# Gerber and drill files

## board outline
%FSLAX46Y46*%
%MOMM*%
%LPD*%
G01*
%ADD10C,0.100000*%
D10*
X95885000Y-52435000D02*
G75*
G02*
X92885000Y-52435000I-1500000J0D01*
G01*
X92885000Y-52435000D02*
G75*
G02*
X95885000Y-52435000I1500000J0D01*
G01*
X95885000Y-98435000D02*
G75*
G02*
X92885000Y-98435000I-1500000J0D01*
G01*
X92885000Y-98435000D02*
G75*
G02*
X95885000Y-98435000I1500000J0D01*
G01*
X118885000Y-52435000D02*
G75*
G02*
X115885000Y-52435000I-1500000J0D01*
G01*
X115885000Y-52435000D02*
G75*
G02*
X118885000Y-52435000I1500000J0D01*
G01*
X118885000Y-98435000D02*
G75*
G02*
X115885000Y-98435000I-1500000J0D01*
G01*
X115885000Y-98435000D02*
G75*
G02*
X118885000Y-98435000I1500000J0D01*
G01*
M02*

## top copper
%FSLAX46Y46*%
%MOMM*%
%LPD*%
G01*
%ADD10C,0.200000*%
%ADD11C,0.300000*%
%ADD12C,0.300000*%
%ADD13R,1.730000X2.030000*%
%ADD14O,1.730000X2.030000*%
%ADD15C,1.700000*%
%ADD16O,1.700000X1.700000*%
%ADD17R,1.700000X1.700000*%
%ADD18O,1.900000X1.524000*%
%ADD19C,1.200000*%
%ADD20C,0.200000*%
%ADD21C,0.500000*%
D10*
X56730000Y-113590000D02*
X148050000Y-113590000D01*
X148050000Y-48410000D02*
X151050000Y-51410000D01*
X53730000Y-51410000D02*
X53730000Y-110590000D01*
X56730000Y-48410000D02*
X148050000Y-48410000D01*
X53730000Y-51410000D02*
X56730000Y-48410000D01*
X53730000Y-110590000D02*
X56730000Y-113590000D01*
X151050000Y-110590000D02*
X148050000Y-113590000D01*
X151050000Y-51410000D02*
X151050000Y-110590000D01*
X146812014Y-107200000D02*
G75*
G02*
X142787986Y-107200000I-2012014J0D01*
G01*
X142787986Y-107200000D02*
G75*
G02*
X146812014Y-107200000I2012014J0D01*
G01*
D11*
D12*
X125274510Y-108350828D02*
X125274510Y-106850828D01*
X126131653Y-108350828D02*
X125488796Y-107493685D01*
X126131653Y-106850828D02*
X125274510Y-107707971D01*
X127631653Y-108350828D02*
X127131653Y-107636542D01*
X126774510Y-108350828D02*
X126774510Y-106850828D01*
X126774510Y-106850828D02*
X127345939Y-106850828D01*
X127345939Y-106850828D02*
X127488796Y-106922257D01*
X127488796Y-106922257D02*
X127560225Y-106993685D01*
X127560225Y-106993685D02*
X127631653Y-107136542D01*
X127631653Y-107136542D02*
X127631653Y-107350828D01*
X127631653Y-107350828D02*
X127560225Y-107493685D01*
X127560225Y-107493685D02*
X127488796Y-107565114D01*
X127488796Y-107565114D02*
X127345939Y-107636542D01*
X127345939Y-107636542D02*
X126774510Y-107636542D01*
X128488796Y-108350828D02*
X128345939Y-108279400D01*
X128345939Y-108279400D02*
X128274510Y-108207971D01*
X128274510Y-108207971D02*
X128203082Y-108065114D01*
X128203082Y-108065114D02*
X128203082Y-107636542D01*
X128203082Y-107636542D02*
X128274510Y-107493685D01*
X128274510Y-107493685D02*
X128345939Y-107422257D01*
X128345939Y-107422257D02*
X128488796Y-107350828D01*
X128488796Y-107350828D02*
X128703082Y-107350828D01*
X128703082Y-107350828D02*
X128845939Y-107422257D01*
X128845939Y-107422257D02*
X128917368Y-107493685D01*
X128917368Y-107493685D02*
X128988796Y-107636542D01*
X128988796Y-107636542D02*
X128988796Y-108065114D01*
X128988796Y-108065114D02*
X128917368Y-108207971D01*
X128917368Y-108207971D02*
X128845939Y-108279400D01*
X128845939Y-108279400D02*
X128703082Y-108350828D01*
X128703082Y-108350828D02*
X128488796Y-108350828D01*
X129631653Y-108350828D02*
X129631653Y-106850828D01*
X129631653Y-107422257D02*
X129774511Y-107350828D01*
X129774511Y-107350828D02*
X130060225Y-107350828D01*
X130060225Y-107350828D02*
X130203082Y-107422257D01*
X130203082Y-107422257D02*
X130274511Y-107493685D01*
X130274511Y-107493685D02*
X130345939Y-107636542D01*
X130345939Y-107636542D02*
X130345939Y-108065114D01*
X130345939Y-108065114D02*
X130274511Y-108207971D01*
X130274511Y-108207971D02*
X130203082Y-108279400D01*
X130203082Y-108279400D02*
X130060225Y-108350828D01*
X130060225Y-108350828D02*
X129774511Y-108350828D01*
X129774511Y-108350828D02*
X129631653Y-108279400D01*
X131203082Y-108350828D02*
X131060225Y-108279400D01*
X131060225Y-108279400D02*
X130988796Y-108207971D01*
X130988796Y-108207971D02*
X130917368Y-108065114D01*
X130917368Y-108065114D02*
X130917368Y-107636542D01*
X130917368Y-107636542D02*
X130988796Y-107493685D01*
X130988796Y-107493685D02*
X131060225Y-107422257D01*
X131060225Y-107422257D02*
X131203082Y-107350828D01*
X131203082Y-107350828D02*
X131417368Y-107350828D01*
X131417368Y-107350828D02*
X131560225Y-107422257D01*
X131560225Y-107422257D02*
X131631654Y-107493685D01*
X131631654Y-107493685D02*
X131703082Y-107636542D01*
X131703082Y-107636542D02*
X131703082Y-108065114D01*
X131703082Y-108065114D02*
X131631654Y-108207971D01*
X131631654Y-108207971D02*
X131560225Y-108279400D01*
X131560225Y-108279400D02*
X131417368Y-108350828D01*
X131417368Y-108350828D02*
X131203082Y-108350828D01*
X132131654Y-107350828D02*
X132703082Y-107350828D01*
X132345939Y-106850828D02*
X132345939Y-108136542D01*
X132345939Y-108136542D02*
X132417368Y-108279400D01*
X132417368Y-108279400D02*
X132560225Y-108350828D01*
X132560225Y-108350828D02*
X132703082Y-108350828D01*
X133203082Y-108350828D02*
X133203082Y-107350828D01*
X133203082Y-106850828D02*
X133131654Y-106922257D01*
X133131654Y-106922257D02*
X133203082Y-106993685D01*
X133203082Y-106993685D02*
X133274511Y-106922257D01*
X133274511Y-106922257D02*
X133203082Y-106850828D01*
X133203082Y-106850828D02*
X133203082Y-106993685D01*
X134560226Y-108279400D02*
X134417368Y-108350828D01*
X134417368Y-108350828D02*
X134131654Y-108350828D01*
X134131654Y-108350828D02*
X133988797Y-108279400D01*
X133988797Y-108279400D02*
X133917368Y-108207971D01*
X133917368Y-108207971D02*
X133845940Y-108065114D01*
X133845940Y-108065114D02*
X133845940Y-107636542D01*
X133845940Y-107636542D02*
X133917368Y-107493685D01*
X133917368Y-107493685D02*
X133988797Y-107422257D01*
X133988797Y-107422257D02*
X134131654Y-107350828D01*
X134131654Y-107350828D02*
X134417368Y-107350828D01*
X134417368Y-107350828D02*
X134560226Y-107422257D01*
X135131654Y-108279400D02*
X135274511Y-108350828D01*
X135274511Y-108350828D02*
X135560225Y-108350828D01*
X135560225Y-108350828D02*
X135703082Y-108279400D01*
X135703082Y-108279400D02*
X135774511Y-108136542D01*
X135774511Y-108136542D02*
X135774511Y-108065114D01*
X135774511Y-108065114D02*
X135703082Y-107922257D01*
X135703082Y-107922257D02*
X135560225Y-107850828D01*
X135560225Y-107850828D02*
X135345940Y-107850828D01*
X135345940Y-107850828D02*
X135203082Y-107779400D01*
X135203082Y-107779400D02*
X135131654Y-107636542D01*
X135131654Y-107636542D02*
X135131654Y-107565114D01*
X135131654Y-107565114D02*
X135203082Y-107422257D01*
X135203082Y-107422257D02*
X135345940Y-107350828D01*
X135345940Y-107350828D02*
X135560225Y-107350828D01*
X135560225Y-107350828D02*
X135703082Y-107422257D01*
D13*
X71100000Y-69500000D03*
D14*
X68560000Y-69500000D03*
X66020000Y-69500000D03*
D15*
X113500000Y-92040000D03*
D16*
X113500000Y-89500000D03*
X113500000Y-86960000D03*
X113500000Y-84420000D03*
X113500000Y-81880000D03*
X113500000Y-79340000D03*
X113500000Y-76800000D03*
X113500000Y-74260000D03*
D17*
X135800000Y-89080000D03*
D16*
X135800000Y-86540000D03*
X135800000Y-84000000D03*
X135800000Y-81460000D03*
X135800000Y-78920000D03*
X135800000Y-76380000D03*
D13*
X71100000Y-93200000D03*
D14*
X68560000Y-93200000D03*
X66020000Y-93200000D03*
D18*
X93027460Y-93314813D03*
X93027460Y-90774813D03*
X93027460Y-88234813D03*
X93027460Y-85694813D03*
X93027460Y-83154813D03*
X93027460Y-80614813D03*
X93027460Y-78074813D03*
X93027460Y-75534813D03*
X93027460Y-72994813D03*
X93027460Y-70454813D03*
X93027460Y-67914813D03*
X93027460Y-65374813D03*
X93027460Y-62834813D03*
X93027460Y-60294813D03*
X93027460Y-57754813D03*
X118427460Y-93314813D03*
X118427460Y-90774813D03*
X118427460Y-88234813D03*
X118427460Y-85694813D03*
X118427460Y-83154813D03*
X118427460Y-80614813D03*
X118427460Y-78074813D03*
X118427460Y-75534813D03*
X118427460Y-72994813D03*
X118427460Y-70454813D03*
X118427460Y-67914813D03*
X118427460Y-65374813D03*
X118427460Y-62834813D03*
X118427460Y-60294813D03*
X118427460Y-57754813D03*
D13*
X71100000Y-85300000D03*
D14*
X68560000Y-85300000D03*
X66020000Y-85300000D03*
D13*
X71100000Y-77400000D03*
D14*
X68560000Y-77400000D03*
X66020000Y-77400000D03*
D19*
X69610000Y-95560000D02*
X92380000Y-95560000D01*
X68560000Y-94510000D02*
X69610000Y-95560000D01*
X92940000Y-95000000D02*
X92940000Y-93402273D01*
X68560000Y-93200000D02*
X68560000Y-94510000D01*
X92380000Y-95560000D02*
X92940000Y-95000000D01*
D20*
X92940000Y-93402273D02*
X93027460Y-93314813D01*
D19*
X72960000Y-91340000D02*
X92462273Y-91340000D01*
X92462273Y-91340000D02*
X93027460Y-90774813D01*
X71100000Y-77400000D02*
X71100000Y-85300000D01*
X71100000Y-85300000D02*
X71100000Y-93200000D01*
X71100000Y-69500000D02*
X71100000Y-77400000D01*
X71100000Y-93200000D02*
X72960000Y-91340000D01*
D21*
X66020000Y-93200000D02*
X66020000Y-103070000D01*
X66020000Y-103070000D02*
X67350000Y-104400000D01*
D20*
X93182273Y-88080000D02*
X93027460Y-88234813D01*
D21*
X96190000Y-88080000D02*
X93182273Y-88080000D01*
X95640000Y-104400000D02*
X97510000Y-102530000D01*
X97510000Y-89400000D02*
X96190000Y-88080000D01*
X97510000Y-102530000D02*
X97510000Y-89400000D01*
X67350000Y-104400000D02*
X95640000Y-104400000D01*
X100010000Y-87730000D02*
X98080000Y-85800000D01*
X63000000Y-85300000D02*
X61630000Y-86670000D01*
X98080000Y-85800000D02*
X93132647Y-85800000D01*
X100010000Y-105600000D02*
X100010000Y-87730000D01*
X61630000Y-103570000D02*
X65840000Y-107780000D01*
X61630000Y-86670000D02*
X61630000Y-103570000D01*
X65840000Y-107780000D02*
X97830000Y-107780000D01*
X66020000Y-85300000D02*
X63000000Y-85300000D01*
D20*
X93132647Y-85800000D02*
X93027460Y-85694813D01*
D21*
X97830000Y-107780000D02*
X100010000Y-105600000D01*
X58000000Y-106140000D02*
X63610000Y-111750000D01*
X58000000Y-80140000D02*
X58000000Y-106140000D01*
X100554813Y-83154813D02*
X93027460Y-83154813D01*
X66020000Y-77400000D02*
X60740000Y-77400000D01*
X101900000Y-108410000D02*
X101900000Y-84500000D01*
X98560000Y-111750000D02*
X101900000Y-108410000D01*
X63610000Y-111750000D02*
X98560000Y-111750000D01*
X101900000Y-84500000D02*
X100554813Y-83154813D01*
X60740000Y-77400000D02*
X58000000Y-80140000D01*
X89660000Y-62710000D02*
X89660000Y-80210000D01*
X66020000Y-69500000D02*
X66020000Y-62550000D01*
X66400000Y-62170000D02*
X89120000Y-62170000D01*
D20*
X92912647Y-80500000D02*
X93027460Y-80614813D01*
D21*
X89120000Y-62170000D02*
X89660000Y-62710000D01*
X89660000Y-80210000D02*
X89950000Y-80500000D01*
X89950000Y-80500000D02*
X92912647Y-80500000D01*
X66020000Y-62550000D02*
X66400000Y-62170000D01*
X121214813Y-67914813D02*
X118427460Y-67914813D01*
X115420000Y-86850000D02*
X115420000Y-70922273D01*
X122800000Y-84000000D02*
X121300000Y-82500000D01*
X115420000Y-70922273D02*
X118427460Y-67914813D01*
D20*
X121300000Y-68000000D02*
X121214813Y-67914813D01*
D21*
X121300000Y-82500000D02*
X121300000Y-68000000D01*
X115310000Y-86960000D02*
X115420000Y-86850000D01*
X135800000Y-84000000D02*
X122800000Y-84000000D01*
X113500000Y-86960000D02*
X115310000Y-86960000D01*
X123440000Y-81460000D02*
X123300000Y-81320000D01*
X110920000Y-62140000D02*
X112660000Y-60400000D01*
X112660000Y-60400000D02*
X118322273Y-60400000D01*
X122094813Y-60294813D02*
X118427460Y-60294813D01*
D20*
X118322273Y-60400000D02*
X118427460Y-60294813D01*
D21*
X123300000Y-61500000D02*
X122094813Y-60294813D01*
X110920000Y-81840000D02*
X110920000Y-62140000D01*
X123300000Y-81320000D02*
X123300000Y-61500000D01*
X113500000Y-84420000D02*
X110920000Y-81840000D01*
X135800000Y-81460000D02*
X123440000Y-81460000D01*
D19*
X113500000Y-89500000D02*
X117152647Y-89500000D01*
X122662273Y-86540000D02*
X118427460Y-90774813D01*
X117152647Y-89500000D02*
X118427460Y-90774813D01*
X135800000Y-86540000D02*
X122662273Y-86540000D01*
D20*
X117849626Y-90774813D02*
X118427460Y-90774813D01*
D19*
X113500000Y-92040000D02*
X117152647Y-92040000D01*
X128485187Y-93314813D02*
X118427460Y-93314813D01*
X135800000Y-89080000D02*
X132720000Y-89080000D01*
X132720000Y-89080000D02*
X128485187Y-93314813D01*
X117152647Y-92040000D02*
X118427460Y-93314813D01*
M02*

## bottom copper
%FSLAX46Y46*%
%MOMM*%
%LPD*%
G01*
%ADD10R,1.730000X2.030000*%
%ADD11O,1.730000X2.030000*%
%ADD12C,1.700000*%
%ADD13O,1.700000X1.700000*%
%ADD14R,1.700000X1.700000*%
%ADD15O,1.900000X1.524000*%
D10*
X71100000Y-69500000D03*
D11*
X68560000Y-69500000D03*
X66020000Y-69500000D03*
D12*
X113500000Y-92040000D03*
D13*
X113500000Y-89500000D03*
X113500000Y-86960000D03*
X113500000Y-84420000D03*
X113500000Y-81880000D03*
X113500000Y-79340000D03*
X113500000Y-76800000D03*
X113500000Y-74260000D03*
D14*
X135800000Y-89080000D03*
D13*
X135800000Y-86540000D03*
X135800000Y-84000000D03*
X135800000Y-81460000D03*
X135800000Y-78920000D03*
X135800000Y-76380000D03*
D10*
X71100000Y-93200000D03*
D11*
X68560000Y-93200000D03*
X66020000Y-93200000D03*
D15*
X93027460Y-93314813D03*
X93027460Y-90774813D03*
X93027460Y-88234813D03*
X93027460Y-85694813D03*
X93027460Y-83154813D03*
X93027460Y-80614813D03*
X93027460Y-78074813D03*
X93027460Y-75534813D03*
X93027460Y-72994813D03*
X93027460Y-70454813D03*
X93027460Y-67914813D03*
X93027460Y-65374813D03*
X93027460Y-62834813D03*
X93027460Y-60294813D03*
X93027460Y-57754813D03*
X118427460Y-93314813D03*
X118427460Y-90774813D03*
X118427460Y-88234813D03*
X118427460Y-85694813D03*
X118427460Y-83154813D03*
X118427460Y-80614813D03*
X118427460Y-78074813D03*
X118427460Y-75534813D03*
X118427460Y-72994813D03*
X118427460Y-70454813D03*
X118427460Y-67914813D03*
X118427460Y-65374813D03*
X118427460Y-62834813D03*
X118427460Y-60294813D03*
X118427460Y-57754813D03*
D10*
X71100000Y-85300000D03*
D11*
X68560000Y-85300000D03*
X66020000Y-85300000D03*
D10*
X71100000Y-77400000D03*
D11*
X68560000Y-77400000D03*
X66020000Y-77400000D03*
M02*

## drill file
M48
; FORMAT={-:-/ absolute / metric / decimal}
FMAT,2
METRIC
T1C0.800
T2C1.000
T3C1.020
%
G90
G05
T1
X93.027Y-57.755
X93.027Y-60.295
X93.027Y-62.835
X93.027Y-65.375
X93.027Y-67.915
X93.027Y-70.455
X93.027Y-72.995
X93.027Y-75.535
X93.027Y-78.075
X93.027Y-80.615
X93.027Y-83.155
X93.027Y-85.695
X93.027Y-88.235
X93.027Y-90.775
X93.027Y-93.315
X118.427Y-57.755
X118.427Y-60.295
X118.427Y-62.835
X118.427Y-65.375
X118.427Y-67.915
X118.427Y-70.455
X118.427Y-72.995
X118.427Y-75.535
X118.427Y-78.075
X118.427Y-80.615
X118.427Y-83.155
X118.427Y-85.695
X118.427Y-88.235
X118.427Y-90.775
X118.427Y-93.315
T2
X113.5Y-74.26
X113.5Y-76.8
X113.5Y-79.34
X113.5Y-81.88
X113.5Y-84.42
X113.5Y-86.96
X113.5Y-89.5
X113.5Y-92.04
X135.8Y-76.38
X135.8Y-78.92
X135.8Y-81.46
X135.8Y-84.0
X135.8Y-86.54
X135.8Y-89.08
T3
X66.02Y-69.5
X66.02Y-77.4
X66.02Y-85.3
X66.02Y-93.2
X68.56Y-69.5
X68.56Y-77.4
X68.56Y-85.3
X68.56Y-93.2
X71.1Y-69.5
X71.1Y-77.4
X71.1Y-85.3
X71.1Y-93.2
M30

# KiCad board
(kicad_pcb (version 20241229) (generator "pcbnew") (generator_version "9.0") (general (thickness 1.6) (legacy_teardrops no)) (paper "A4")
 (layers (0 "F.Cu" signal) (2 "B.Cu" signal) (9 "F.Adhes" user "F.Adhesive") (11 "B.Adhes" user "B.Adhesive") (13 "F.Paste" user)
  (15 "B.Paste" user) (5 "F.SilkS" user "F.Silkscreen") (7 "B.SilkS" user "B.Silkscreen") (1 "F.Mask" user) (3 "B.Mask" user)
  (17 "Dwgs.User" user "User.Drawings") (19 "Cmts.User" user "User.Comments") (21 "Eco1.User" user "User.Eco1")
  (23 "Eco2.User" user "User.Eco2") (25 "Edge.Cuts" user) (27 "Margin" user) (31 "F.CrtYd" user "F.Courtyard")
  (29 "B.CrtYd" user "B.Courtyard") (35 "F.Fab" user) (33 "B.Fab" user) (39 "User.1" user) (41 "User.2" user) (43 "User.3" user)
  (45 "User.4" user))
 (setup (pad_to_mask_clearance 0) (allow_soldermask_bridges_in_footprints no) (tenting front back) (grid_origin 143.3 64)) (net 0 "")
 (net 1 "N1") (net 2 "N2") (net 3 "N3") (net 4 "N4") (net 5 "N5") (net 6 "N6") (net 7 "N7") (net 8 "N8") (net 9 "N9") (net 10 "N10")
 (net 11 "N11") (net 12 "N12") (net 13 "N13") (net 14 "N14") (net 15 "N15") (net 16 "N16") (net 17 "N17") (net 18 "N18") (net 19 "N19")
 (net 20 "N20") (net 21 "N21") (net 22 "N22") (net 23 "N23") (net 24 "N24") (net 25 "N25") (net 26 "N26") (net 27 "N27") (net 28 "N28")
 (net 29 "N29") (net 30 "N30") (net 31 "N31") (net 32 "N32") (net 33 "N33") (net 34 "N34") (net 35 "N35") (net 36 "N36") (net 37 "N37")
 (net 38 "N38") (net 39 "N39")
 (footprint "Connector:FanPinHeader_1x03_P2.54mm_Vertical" (layer "F.Cu") (at 71.1 69.5 180)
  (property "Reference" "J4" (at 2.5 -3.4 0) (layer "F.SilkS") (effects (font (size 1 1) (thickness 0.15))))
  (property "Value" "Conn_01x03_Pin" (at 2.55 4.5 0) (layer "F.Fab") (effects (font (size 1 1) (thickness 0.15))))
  (pad "1" thru_hole rect (at 0 0 270) (size 2.03 1.73) (drill 1.02) (layers "*.Cu" "*.Mask") (remove_unused_layers no) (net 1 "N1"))
  (pad "2" thru_hole oval (at 2.54 0 270) (size 2.03 1.73) (drill 1.02) (layers "*.Cu" "*.Mask") (remove_unused_layers no) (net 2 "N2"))
  (pad "3" thru_hole oval (at 5.08 0 270) (size 2.03 1.73) (drill 1.02) (layers "*.Cu" "*.Mask") (remove_unused_layers no) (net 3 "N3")))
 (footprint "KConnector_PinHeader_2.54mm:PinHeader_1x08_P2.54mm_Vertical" (layer "F.Cu") (at 113.5 92.04 180)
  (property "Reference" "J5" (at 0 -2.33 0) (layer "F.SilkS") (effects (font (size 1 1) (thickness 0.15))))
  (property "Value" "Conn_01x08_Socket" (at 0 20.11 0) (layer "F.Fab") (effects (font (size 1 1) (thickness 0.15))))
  (pad "1" thru_hole circle (at 0 0 180) (size 1.7 1.7) (drill 1) (layers "*.Cu" "*.Mask") (remove_unused_layers no) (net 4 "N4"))
  (pad "2" thru_hole oval (at 0 2.54 180) (size 1.7 1.7) (drill 1) (layers "*.Cu" "*.Mask") (remove_unused_layers no) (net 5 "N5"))
  (pad "3" thru_hole oval (at 0 5.08 180) (size 1.7 1.7) (drill 1) (layers "*.Cu" "*.Mask") (remove_unused_layers no) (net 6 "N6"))
  (pad "4" thru_hole oval (at 0 7.62 180) (size 1.7 1.7) (drill 1) (layers "*.Cu" "*.Mask") (remove_unused_layers no) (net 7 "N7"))
  (pad "5" thru_hole oval (at 0 10.16 180) (size 1.7 1.7) (drill 1) (layers "*.Cu" "*.Mask") (remove_unused_layers no) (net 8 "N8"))
  (pad "6" thru_hole oval (at 0 12.7 180) (size 1.7 1.7) (drill 1) (layers "*.Cu" "*.Mask") (remove_unused_layers no) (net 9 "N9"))
  (pad "7" thru_hole oval (at 0 15.24 180) (size 1.7 1.7) (drill 1) (layers "*.Cu" "*.Mask") (remove_unused_layers no) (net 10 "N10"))
  (pad "8" thru_hole oval (at 0 17.78 180) (size 1.7 1.7) (drill 1) (layers "*.Cu" "*.Mask") (remove_unused_layers no) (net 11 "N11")))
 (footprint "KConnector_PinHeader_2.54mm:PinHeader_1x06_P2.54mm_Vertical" (layer "F.Cu") (at 135.8 89.08 180)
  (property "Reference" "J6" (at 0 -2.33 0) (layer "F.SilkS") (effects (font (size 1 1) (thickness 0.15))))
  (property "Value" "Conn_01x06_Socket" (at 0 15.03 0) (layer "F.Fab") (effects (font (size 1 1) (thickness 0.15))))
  (pad "1" thru_hole rect (at 0 0 180) (size 1.7 1.7) (drill 1) (layers "*.Cu" "*.Mask") (remove_unused_layers no) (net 4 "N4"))
  (pad "2" thru_hole oval (at 0 2.54 180) (size 1.7 1.7) (drill 1) (layers "*.Cu" "*.Mask") (remove_unused_layers no) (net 5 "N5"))
  (pad "3" thru_hole oval (at 0 5.08 180) (size 1.7 1.7) (drill 1) (layers "*.Cu" "*.Mask") (remove_unused_layers no) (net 6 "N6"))
  (pad "4" thru_hole oval (at 0 7.62 180) (size 1.7 1.7) (drill 1) (layers "*.Cu" "*.Mask") (remove_unused_layers no) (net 7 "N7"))
  (pad "5" thru_hole oval (at 0 10.16 180) (size 1.7 1.7) (drill 1) (layers "*.Cu" "*.Mask") (remove_unused_layers no) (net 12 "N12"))
  (pad "6" thru_hole oval (at 0 12.7 180) (size 1.7 1.7) (drill 1) (layers "*.Cu" "*.Mask") (remove_unused_layers no) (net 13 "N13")))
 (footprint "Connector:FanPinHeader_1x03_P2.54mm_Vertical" (layer "F.Cu") (at 71.1 93.2 180)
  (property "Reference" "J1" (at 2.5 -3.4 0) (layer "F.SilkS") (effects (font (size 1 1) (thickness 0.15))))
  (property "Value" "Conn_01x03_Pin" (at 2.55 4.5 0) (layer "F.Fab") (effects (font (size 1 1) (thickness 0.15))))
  (pad "1" thru_hole rect (at 0 0 270) (size 2.03 1.73) (drill 1.02) (layers "*.Cu" "*.Mask") (remove_unused_layers no) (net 1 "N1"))
  (pad "2" thru_hole oval (at 2.54 0 270) (size 2.03 1.73) (drill 1.02) (layers "*.Cu" "*.Mask") (remove_unused_layers no) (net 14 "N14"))
  (pad "3" thru_hole oval (at 5.08 0 270) (size 2.03 1.73) (drill 1.02) (layers "*.Cu" "*.Mask") (remove_unused_layers no) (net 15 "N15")))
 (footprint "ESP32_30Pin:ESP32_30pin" (layer "F.Cu") (at 104.955 76.295)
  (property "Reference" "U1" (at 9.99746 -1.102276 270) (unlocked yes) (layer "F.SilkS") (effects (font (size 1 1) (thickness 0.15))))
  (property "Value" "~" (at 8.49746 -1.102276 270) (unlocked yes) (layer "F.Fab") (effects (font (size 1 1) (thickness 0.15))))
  (fp_circle (center -10.57 -23.86) (end -10.57 -22.36) (stroke (width 0.1) (type default)) (fill no) (layer "Edge.Cuts"))
  (fp_circle (center -10.57 22.14) (end -10.57 23.64) (stroke (width 0.1) (type default)) (fill no) (layer "Edge.Cuts"))
  (fp_circle (center 12.43 -23.86) (end 12.43 -22.36) (stroke (width 0.1) (type default)) (fill no) (layer "Edge.Cuts"))
  (fp_circle (center 12.43 22.14) (end 12.43 23.64) (stroke (width 0.1) (type default)) (fill no) (layer "Edge.Cuts"))
  (pad "1" thru_hole oval (at -11.92754 17.019813 270) (size 1.524 1.9) (drill 0.8) (layers "*.Cu" "*.Mask") (remove_unused_layers no)
   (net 14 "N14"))
  (pad "2" thru_hole oval (at -11.92754 14.479813 270) (size 1.524 1.9) (drill 0.8) (layers "*.Cu" "*.Mask") (remove_unused_layers no)
   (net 1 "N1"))
  (pad "3" thru_hole oval (at -11.92754 11.939813 270) (size 1.524 1.9) (drill 0.8) (layers "*.Cu" "*.Mask") (remove_unused_layers no)
   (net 15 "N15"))
  (pad "4" thru_hole oval (at -11.92754 9.399813 270) (size 1.524 1.9) (drill 0.8) (layers "*.Cu" "*.Mask") (remove_unused_layers no)
   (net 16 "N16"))
  (pad "5" thru_hole oval (at -11.92754 6.859813 270) (size 1.524 1.9) (drill 0.8) (layers "*.Cu" "*.Mask") (remove_unused_layers no)
   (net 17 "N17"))
  (pad "6" thru_hole oval (at -11.92754 4.319813 270) (size 1.524 1.9) (drill 0.8) (layers "*.Cu" "*.Mask") (remove_unused_layers no)
   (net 3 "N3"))
  (pad "7" thru_hole oval (at -11.92754 1.779813 270) (size 1.524 1.9) (drill 0.8) (layers "*.Cu" "*.Mask") (remove_unused_layers no)
   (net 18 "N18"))
  (pad "8" thru_hole oval (at -11.92754 -0.760187 270) (size 1.524 1.9) (drill 0.8) (layers "*.Cu" "*.Mask") (remove_unused_layers no)
   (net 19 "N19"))
  (pad "9" thru_hole oval (at -11.92754 -3.300187 270) (size 1.524 1.9) (drill 0.8) (layers "*.Cu" "*.Mask") (remove_unused_layers no)
   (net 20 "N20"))
  (pad "10" thru_hole oval (at -11.92754 -5.840187 270) (size 1.524 1.9) (drill 0.8) (layers "*.Cu" "*.Mask") (remove_unused_layers no)
   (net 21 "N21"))
  (pad "11" thru_hole oval (at -11.92754 -8.380187 270) (size 1.524 1.9) (drill 0.8) (layers "*.Cu" "*.Mask") (remove_unused_layers no)
   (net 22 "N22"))
  (pad "12" thru_hole oval (at -11.92754 -10.920187 270) (size 1.524 1.9) (drill 0.8) (layers "*.Cu" "*.Mask") (remove_unused_layers no)
   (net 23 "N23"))
  (pad "13" thru_hole oval (at -11.92754 -13.460187 270) (size 1.524 1.9) (drill 0.8) (layers "*.Cu" "*.Mask") (remove_unused_layers no)
   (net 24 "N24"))
  (pad "14" thru_hole oval (at -11.92754 -16.000187 270) (size 1.524 1.9) (drill 0.8) (layers "*.Cu" "*.Mask") (remove_unused_layers no)
   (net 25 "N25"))
  (pad "15" thru_hole oval (at -11.92754 -18.540187 270) (size 1.524 1.9) (drill 0.8) (layers "*.Cu" "*.Mask") (remove_unused_layers no)
   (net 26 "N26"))
  (pad "16" thru_hole oval (at 13.47246 17.019813 270) (size 1.524 1.9) (drill 0.8) (layers "*.Cu" "*.Mask") (remove_unused_layers no)
   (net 4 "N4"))
  (pad "17" thru_hole oval (at 13.47246 14.479813 270) (size 1.524 1.9) (drill 0.8) (layers "*.Cu" "*.Mask") (remove_unused_layers no)
   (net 5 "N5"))
  (pad "18" thru_hole oval (at 13.47246 11.939813 270) (size 1.524 1.9) (drill 0.8) (layers "*.Cu" "*.Mask") (remove_unused_layers no)
   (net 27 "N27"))
  (pad "19" thru_hole oval (at 13.47246 9.399813 270) (size 1.524 1.9) (drill 0.8) (layers "*.Cu" "*.Mask") (remove_unused_layers no)
   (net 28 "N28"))
  (pad "20" thru_hole oval (at 13.47246 6.859813 270) (size 1.524 1.9) (drill 0.8) (layers "*.Cu" "*.Mask" "Dwgs.User")
   (remove_unused_layers no) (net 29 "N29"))
  (pad "21" thru_hole oval (at 13.47246 4.319813 270) (size 1.524 1.9) (drill 0.8) (layers "*.Cu" "*.Mask") (remove_unused_layers no)
   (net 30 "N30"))
  (pad "22" thru_hole oval (at 13.47246 1.779813 270) (size 1.524 1.9) (drill 0.8) (layers "*.Cu" "*.Mask") (remove_unused_layers no)
   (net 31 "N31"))
  (pad "23" thru_hole oval (at 13.47246 -0.760187 270) (size 1.524 1.9) (drill 0.8) (layers "*.Cu" "*.Mask") (remove_unused_layers no)
   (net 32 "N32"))
  (pad "24" thru_hole oval (at 13.47246 -3.300187 270) (size 1.524 1.9) (drill 0.8) (layers "*.Cu" "*.Mask") (remove_unused_layers no)
   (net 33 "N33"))
  (pad "25" thru_hole oval (at 13.47246 -5.840187 270) (size 1.524 1.9) (drill 0.8) (layers "*.Cu" "*.Mask") (remove_unused_layers no)
   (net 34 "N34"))
  (pad "26" thru_hole oval (at 13.47246 -8.380187 270) (size 1.524 1.9) (drill 0.8) (layers "*.Cu" "*.Mask") (remove_unused_layers no)
   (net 6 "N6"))
  (pad "27" thru_hole oval (at 13.47246 -10.920187 270) (size 1.524 1.9) (drill 0.8) (layers "*.Cu" "*.Mask") (remove_unused_layers no)
   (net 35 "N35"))
  (pad "28" thru_hole oval (at 13.47246 -13.460187 270) (size 1.524 1.9) (drill 0.8) (layers "*.Cu" "*.Mask") (remove_unused_layers no)
   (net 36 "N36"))
  (pad "29" thru_hole oval (at 13.47246 -16.000187 270) (size 1.524 1.9) (drill 0.8) (layers "*.Cu" "*.Mask") (remove_unused_layers no)
   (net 7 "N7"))
  (pad "30" thru_hole oval (at 13.47246 -18.540187 270) (size 1.524 1.9) (drill 0.8) (layers "*.Cu" "*.Mask") (remove_unused_layers no)
   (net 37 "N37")))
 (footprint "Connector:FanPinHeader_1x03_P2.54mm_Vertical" (layer "F.Cu") (at 71.1 85.3 180)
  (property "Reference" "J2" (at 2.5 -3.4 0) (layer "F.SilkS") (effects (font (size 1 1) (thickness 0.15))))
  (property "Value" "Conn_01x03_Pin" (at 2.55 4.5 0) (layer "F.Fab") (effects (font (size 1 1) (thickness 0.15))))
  (pad "1" thru_hole rect (at 0 0 270) (size 2.03 1.73) (drill 1.02) (layers "*.Cu" "*.Mask") (remove_unused_layers no) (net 1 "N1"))
  (pad "2" thru_hole oval (at 2.54 0 270) (size 2.03 1.73) (drill 1.02) (layers "*.Cu" "*.Mask") (remove_unused_layers no) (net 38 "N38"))
  (pad "3" thru_hole oval (at 5.08 0 270) (size 2.03 1.73) (drill 1.02) (layers "*.Cu" "*.Mask") (remove_unused_layers no) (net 16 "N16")))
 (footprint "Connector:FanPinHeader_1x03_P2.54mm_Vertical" (layer "F.Cu") (at 71.1 77.4 180)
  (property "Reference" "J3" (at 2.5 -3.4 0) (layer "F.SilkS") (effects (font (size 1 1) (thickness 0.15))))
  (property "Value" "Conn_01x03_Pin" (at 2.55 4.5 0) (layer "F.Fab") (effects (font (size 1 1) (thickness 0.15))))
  (pad "1" thru_hole rect (at 0 0 270) (size 2.03 1.73) (drill 1.02) (layers "*.Cu" "*.Mask") (remove_unused_layers no) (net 1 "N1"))
  (pad "2" thru_hole oval (at 2.54 0 270) (size 2.03 1.73) (drill 1.02) (layers "*.Cu" "*.Mask") (remove_unused_layers no) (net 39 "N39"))
  (pad "3" thru_hole oval (at 5.08 0 270) (size 2.03 1.73) (drill 1.02) (layers "*.Cu" "*.Mask") (remove_unused_layers no) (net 17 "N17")))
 (gr_line (start 56.73 113.59) (end 148.05 113.59) (stroke (width 0.2) (type default)) (layer "F.Cu"))
 (gr_line (start 148.05 48.41) (end 151.05 51.41) (stroke (width 0.2) (type default)) (layer "F.Cu"))
 (gr_line (start 53.73 51.41) (end 53.73 110.59) (stroke (width 0.2) (type default)) (layer "F.Cu"))
 (gr_line (start 56.73 48.41) (end 148.05 48.41) (stroke (width 0.2) (type default)) (layer "F.Cu"))
 (gr_line (start 53.73 51.41) (end 56.73 48.41) (stroke (width 0.2) (type default)) (layer "F.Cu"))
 (gr_line (start 53.73 110.59) (end 56.73 113.59) (stroke (width 0.2) (type default)) (layer "F.Cu"))
 (gr_line (start 151.05 110.59) (end 148.05 113.59) (stroke (width 0.2) (type default)) (layer "F.Cu"))
 (gr_line (start 151.05 51.41) (end 151.05 110.59) (stroke (width 0.2) (type default)) (layer "F.Cu"))
 (gr_circle (center 144.8 107.2) (end 146.81 107.11) (stroke (width 0.2) (type default)) (fill no) (layer "F.Cu"))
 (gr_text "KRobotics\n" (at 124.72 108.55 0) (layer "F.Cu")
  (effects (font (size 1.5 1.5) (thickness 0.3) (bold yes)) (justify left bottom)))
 (segment (start 69.61 95.56) (end 92.38 95.56) (width 1.2) (layer "F.Cu") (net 14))
 (segment (start 68.56 94.51) (end 69.61 95.56) (width 1.2) (layer "F.Cu") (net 14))
 (segment (start 92.94 95) (end 92.94 93.402273) (width 1.2) (layer "F.Cu") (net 14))
 (segment (start 68.56 93.2) (end 68.56 94.51) (width 1.2) (layer "F.Cu") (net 14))
 (segment (start 92.38 95.56) (end 92.94 95) (width 1.2) (layer "F.Cu") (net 14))
 (segment (start 92.94 93.402273) (end 93.02746 93.314813) (width 0.2) (layer "F.Cu") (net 14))
 (segment (start 72.96 91.34) (end 92.462273 91.34) (width 1.2) (layer "F.Cu") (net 1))
 (segment (start 92.462273 91.34) (end 93.02746 90.774813) (width 1.2) (layer "F.Cu") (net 1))
 (segment (start 71.1 77.4) (end 71.1 85.3) (width 1.2) (layer "F.Cu") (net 1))
 (segment (start 71.1 85.3) (end 71.1 93.2) (width 1.2) (layer "F.Cu") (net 1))
 (segment (start 71.1 69.5) (end 71.1 77.4) (width 1.2) (layer "F.Cu") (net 1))
 (segment (start 71.1 93.2) (end 72.96 91.34) (width 1.2) (layer "F.Cu") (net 1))
 (segment (start 66.02 93.2) (end 66.02 103.07) (width 0.5) (layer "F.Cu") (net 15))
 (segment (start 66.02 103.07) (end 67.35 104.4) (width 0.5) (layer "F.Cu") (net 15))
 (segment (start 93.182273 88.08) (end 93.02746 88.234813) (width 0.2) (layer "F.Cu") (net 15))
 (segment (start 96.19 88.08) (end 93.182273 88.08) (width 0.5) (layer "F.Cu") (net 15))
 (segment (start 95.64 104.4) (end 97.51 102.53) (width 0.5) (layer "F.Cu") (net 15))
 (segment (start 97.51 89.4) (end 96.19 88.08) (width 0.5) (layer "F.Cu") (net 15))
 (segment (start 97.51 102.53) (end 97.51 89.4) (width 0.5) (layer "F.Cu") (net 15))
 (segment (start 67.35 104.4) (end 95.64 104.4) (width 0.5) (layer "F.Cu") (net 15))
 (segment (start 100.01 87.73) (end 98.08 85.8) (width 0.5) (layer "F.Cu") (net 16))
 (segment (start 63 85.3) (end 61.63 86.67) (width 0.5) (layer "F.Cu") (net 16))
 (segment (start 98.08 85.8) (end 93.132647 85.8) (width 0.5) (layer "F.Cu") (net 16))
 (segment (start 100.01 105.6) (end 100.01 87.73) (width 0.5) (layer "F.Cu") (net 16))
 (segment (start 61.63 103.57) (end 65.84 107.78) (width 0.5) (layer "F.Cu") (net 16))
 (segment (start 61.63 86.67) (end 61.63 103.57) (width 0.5) (layer "F.Cu") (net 16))
 (segment (start 65.84 107.78) (end 97.83 107.78) (width 0.5) (layer "F.Cu") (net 16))
 (segment (start 66.02 85.3) (end 63 85.3) (width 0.5) (layer "F.Cu") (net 16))
 (segment (start 93.132647 85.8) (end 93.02746 85.694813) (width 0.2) (layer "F.Cu") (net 16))
 (segment (start 97.83 107.78) (end 100.01 105.6) (width 0.5) (layer "F.Cu") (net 16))
 (segment (start 58 106.14) (end 63.61 111.75) (width 0.5) (layer "F.Cu") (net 17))
 (segment (start 58 80.14) (end 58 106.14) (width 0.5) (layer "F.Cu") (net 17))
 (segment (start 100.554813 83.154813) (end 93.02746 83.154813) (width 0.5) (layer "F.Cu") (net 17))
 (segment (start 66.02 77.4) (end 60.74 77.4) (width 0.5) (layer "F.Cu") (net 17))
 (segment (start 101.9 108.41) (end 101.9 84.5) (width 0.5) (layer "F.Cu") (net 17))
 (segment (start 98.56 111.75) (end 101.9 108.41) (width 0.5) (layer "F.Cu") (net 17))
 (segment (start 63.61 111.75) (end 98.56 111.75) (width 0.5) (layer "F.Cu") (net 17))
 (segment (start 101.9 84.5) (end 100.554813 83.154813) (width 0.5) (layer "F.Cu") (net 17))
 (segment (start 60.74 77.4) (end 58 80.14) (width 0.5) (layer "F.Cu") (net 17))
 (segment (start 89.66 62.71) (end 89.66 80.21) (width 0.5) (layer "F.Cu") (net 3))
 (segment (start 66.02 69.5) (end 66.02 62.55) (width 0.5) (layer "F.Cu") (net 3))
 (segment (start 66.4 62.17) (end 89.12 62.17) (width 0.5) (layer "F.Cu") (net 3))
 (segment (start 92.912647 80.5) (end 93.02746 80.614813) (width 0.2) (layer "F.Cu") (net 3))
 (segment (start 89.12 62.17) (end 89.66 62.71) (width 0.5) (layer "F.Cu") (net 3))
 (segment (start 89.66 80.21) (end 89.95 80.5) (width 0.5) (layer "F.Cu") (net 3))
 (segment (start 89.95 80.5) (end 92.912647 80.5) (width 0.5) (layer "F.Cu") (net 3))
 (segment (start 66.02 62.55) (end 66.4 62.17) (width 0.5) (layer "F.Cu") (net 3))
 (segment (start 121.214813 67.914813) (end 118.42746 67.914813) (width 0.5) (layer "F.Cu") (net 6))
 (segment (start 115.42 86.85) (end 115.42 70.922273) (width 0.5) (layer "F.Cu") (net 6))
 (segment (start 122.8 84) (end 121.3 82.5) (width 0.5) (layer "F.Cu") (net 6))
 (segment (start 115.42 70.922273) (end 118.42746 67.914813) (width 0.5) (layer "F.Cu") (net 6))
 (segment (start 121.3 68) (end 121.214813 67.914813) (width 0.2) (layer "F.Cu") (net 6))
 (segment (start 121.3 82.5) (end 121.3 68) (width 0.5) (layer "F.Cu") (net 6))
 (segment (start 115.31 86.96) (end 115.42 86.85) (width 0.5) (layer "F.Cu") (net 6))
 (segment (start 135.8 84) (end 122.8 84) (width 0.5) (layer "F.Cu") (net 6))
 (segment (start 113.5 86.96) (end 115.31 86.96) (width 0.5) (layer "F.Cu") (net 6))
 (segment (start 123.44 81.46) (end 123.3 81.32) (width 0.5) (layer "F.Cu") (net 7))
 (segment (start 110.92 62.14) (end 112.66 60.4) (width 0.5) (layer "F.Cu") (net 7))
 (segment (start 112.66 60.4) (end 118.322273 60.4) (width 0.5) (layer "F.Cu") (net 7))
 (segment (start 122.094813 60.294813) (end 118.42746 60.294813) (width 0.5) (layer "F.Cu") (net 7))
 (segment (start 118.322273 60.4) (end 118.42746 60.294813) (width 0.2) (layer "F.Cu") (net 7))
 (segment (start 123.3 61.5) (end 122.094813 60.294813) (width 0.5) (layer "F.Cu") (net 7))
 (segment (start 110.92 81.84) (end 110.92 62.14) (width 0.5) (layer "F.Cu") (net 7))
 (segment (start 123.3 81.32) (end 123.3 61.5) (width 0.5) (layer "F.Cu") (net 7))
 (segment (start 113.5 84.42) (end 110.92 81.84) (width 0.5) (layer "F.Cu") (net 7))
 (segment (start 135.8 81.46) (end 123.44 81.46) (width 0.5) (layer "F.Cu") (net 7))
 (segment (start 113.5 89.5) (end 117.152647 89.5) (width 1.2) (layer "F.Cu") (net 5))
 (segment (start 122.662273 86.54) (end 118.42746 90.774813) (width 1.2) (layer "F.Cu") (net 5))
 (segment (start 117.152647 89.5) (end 118.42746 90.774813) (width 1.2) (layer "F.Cu") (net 5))
 (segment (start 135.8 86.54) (end 122.662273 86.54) (width 1.2) (layer "F.Cu") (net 5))
 (segment (start 117.849626 90.774813) (end 118.42746 90.774813) (width 0.2) (layer "F.Cu") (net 5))
 (segment (start 113.5 92.04) (end 117.152647 92.04) (width 1.2) (layer "F.Cu") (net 4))
 (segment (start 128.485187 93.314813) (end 118.42746 93.314813) (width 1.2) (layer "F.Cu") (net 4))
 (segment (start 135.8 89.08) (end 132.72 89.08) (width 1.2) (layer "F.Cu") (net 4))
 (segment (start 132.72 89.08) (end 128.485187 93.314813) (width 1.2) (layer "F.Cu") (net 4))
 (segment (start 117.152647 92.04) (end 118.42746 93.314813) (width 1.2) (layer "F.Cu") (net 4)))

